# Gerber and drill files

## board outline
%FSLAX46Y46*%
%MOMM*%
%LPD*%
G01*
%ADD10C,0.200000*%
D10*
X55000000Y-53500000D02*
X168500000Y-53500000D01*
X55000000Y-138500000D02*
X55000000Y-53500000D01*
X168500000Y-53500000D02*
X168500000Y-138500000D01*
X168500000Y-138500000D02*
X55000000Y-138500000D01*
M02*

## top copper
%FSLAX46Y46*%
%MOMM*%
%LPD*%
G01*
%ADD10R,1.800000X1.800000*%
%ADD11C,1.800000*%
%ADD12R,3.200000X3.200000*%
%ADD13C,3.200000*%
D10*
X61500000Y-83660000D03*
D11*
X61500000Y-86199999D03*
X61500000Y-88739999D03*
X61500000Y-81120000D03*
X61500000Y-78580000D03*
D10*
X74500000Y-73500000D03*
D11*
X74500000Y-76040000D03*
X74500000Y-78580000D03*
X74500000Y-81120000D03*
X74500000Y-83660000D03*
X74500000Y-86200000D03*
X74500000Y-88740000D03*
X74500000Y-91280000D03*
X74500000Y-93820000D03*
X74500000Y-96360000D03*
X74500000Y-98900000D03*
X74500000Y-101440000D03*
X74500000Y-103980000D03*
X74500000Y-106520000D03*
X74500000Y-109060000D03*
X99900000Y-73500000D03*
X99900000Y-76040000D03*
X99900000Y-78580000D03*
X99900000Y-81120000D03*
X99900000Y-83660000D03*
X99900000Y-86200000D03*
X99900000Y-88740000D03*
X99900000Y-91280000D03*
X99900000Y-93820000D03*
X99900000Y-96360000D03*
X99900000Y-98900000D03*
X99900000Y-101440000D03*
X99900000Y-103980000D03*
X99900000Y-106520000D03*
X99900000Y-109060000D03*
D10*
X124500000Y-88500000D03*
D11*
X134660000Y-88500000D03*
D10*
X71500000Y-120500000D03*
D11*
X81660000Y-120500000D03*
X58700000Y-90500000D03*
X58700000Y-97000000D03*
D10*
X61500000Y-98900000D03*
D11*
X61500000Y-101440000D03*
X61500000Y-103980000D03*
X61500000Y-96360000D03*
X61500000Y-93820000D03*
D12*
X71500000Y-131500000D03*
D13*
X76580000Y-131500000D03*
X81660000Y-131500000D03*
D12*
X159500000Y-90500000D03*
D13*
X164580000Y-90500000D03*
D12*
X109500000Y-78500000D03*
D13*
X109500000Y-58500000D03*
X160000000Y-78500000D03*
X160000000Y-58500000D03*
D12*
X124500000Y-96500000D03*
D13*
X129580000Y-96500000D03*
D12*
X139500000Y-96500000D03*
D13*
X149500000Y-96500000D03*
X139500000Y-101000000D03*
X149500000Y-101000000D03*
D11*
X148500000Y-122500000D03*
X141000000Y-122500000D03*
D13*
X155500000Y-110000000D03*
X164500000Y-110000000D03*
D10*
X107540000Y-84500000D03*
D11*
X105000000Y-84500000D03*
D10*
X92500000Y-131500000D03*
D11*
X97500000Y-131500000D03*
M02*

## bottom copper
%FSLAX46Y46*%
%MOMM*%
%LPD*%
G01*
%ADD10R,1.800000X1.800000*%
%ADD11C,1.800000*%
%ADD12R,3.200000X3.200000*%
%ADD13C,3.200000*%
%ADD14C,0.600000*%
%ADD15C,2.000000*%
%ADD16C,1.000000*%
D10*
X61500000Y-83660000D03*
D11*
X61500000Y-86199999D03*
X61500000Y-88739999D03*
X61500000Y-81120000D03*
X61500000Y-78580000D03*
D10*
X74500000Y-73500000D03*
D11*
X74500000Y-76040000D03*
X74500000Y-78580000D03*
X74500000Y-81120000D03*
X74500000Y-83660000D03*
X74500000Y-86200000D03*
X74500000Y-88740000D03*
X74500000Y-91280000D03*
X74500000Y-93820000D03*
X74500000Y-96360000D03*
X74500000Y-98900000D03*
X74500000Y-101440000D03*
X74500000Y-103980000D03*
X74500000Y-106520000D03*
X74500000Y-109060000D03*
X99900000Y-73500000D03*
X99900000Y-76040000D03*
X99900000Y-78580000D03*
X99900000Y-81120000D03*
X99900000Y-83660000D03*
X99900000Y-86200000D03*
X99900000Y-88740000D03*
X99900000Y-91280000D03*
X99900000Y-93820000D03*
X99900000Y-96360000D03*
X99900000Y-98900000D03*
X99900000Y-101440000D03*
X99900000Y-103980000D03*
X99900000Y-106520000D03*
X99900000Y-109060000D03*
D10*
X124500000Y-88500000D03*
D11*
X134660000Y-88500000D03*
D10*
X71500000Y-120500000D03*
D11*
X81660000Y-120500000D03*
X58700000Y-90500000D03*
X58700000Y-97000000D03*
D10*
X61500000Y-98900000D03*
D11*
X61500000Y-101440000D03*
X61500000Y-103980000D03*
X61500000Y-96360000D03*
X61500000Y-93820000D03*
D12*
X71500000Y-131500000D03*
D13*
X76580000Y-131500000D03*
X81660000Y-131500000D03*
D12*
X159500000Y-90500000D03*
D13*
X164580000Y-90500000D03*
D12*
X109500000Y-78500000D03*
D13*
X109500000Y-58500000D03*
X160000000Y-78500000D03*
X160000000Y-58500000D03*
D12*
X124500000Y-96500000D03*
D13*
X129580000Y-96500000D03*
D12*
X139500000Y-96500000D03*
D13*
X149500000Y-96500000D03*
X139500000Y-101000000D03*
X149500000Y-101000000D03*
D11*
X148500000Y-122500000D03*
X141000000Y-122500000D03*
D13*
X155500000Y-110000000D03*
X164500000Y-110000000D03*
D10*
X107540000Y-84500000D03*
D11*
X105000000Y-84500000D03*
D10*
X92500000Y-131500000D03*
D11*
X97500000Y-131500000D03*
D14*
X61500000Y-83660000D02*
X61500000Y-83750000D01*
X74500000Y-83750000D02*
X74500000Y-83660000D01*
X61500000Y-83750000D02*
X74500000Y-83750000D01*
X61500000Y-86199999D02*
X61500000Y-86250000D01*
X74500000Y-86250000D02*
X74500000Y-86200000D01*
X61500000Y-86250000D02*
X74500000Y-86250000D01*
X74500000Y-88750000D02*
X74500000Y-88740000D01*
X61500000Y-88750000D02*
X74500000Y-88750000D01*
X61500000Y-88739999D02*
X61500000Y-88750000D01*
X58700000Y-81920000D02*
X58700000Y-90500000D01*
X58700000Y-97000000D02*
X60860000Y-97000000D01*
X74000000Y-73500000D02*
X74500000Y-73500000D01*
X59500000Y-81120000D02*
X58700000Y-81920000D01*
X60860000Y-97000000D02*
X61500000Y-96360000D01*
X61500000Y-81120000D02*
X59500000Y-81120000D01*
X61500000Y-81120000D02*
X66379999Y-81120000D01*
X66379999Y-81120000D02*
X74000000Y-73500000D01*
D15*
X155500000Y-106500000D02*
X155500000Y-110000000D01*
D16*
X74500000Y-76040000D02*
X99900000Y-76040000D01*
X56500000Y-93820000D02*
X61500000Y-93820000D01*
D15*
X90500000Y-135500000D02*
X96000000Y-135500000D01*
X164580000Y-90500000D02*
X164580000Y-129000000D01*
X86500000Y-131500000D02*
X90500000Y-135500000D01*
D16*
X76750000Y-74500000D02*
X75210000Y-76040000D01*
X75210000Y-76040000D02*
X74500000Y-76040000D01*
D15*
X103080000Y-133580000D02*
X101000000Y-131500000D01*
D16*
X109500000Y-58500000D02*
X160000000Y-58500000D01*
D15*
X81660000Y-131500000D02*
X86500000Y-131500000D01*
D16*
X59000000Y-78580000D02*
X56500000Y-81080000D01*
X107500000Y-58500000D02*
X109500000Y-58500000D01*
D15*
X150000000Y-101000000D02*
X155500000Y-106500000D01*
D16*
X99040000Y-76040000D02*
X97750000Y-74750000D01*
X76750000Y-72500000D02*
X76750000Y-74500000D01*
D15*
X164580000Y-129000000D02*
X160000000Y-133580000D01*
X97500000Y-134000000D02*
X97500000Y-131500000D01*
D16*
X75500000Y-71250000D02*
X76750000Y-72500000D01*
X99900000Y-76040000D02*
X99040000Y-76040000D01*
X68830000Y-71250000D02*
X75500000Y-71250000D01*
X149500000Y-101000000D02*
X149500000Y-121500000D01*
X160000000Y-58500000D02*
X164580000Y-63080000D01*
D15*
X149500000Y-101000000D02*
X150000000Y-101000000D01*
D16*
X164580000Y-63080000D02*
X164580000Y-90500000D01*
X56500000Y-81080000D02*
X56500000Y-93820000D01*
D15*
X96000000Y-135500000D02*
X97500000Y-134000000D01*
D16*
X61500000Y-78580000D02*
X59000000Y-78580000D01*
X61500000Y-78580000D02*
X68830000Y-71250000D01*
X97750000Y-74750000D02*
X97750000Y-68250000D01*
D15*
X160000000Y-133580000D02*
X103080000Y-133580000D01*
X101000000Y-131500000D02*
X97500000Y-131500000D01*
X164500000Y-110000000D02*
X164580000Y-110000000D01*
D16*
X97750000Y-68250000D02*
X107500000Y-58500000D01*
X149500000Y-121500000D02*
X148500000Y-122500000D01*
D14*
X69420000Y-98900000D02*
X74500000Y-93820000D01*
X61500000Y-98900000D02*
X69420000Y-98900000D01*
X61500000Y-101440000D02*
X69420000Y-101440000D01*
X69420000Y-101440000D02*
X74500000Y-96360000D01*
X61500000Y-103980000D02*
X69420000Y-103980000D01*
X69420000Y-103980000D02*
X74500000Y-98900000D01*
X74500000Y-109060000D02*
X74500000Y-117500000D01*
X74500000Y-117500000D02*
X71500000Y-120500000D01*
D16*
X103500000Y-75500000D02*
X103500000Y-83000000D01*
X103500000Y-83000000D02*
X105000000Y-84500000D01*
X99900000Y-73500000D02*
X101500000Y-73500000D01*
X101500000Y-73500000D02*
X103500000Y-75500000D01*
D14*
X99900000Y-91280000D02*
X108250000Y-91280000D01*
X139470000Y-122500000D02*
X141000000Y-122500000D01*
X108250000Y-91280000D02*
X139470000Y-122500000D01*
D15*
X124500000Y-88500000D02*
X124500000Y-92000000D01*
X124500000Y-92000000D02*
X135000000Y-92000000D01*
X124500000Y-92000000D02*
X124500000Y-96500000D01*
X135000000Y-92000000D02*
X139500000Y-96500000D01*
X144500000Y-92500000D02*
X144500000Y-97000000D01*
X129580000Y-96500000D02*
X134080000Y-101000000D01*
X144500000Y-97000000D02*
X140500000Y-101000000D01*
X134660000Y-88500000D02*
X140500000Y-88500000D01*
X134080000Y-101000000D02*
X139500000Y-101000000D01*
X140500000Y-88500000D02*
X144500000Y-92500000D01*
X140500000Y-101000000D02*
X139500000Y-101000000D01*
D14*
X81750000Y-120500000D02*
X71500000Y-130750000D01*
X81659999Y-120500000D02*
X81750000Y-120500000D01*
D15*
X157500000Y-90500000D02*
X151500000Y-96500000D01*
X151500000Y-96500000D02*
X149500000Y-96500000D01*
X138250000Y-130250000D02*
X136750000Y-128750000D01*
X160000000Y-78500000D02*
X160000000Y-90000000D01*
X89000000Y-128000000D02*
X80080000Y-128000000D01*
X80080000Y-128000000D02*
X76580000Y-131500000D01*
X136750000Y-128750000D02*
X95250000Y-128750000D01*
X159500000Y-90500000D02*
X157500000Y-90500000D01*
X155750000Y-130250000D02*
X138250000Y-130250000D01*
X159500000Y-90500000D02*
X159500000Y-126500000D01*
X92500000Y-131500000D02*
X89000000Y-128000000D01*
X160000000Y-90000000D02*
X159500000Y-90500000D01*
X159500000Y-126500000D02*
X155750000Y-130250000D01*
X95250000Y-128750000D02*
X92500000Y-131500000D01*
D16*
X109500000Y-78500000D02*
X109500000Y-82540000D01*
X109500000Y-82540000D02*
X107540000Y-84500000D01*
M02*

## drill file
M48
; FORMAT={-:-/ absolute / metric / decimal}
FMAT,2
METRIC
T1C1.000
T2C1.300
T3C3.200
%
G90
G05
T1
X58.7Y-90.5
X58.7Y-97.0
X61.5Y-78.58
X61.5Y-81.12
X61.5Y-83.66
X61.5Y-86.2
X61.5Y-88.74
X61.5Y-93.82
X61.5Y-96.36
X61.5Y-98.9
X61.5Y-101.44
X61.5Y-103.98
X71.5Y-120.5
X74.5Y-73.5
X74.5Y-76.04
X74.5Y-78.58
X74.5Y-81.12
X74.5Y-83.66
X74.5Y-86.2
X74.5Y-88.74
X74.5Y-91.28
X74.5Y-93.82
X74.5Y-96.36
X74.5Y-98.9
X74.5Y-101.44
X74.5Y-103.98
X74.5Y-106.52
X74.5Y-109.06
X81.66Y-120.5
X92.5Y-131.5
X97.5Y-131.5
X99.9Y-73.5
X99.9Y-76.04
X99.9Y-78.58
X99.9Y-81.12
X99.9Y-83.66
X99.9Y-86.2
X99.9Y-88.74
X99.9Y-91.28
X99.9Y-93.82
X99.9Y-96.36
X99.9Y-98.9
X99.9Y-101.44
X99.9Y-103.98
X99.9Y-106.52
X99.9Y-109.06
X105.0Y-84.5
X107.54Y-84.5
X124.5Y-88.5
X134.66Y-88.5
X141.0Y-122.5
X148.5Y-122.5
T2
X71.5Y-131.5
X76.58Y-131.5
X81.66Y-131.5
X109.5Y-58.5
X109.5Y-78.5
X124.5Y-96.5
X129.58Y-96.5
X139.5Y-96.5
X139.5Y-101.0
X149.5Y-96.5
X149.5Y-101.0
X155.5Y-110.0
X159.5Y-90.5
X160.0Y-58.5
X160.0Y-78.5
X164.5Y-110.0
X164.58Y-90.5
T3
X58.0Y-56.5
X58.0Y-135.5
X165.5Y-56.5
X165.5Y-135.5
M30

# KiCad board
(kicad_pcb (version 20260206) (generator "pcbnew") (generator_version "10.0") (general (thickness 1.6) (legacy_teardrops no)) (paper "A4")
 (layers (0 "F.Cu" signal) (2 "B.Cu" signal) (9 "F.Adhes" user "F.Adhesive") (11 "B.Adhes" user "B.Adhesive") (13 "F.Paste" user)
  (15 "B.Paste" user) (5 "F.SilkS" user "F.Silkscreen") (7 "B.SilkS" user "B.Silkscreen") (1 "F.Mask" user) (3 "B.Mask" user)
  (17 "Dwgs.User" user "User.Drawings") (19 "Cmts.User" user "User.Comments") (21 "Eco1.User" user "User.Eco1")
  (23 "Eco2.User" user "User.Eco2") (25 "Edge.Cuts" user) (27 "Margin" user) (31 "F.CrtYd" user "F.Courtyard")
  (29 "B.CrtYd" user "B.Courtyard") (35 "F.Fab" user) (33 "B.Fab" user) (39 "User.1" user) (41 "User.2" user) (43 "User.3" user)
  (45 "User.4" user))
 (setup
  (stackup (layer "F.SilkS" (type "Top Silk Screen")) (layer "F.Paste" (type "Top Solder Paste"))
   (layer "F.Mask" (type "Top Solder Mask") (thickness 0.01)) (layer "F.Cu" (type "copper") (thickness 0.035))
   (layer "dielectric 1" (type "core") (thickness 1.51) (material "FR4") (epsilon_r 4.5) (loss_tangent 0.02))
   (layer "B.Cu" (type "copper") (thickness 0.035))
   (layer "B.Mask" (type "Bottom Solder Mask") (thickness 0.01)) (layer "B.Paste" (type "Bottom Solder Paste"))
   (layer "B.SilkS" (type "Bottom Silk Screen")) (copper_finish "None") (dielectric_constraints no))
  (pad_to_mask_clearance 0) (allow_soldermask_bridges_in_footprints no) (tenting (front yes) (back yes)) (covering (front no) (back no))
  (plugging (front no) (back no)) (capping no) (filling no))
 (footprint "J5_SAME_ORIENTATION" (layer "F.Cu") (at 61.5 83.5 -90)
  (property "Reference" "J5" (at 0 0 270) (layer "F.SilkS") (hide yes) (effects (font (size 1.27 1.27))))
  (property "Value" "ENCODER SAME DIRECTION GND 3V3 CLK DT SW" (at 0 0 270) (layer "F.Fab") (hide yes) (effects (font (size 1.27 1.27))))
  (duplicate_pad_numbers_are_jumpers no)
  (pad "1" thru_hole rect (at 0.16 0 270) (size 1.8 1.8) (drill 1) (layers "*.Cu") (remove_unused_layers no) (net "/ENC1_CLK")
   (clearance 0.5) (thermal_bridge_angle 45))
  (pad "2" thru_hole circle (at 2.699999 0 270) (size 1.8 1.8) (drill 1) (layers "*.Cu") (remove_unused_layers no) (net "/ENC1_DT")
   (clearance 0.5))
  (pad "3" thru_hole circle (at 5.239999 0 270) (size 1.8 1.8) (drill 1) (layers "*.Cu") (remove_unused_layers no) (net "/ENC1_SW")
   (clearance 0.5))
  (pad "4" thru_hole circle (at -2.38 0 270) (size 1.8 1.8) (drill 1) (layers "*.Cu") (remove_unused_layers no) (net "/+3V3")
   (clearance 0.5))
  (pad "5" thru_hole circle (at -4.92 0 270) (size 1.8 1.8) (drill 1) (layers "*.Cu") (remove_unused_layers no) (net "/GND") (clearance 0.5)))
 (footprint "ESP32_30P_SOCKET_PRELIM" (layer "F.Cu") (at 74.5 73.5)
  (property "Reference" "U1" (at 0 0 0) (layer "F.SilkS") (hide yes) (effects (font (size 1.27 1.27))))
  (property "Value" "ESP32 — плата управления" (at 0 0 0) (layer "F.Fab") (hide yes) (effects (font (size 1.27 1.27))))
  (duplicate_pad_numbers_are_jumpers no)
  (pad "1" thru_hole rect (at 0 0) (size 1.8 1.8) (drill 1) (layers "*.Cu") (remove_unused_layers no) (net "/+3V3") (clearance 0.5)
   (thermal_bridge_angle 45))
  (pad "2" thru_hole circle (at 0 2.54) (size 1.8 1.8) (drill 1) (layers "*.Cu") (remove_unused_layers no) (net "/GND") (clearance 0.5))
  (pad "3" thru_hole circle (at 0 5.08) (size 1.8 1.8) (drill 1) (layers "*.Cu") (remove_unused_layers no) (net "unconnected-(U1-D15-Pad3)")
   (clearance 0.5))
  (pad "4" thru_hole circle (at 0 7.62) (size 1.8 1.8) (drill 1) (layers "*.Cu") (remove_unused_layers no) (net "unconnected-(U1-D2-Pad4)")
   (clearance 0.5))
  (pad "5" thru_hole circle (at 0 10.16) (size 1.8 1.8) (drill 1) (layers "*.Cu") (remove_unused_layers no) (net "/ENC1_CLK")
   (clearance 0.5))
  (pad "6" thru_hole circle (at 0 12.7) (size 1.8 1.8) (drill 1) (layers "*.Cu") (remove_unused_layers no) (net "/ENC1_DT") (clearance 0.5))
  (pad "7" thru_hole circle (at 0 15.24) (size 1.8 1.8) (drill 1) (layers "*.Cu") (remove_unused_layers no) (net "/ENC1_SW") (clearance 0.5))
  (pad "8" thru_hole circle (at 0 17.78) (size 1.8 1.8) (drill 1) (layers "*.Cu") (remove_unused_layers no) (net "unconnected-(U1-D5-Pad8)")
   (clearance 0.5))
  (pad "9" thru_hole circle (at 0 20.32) (size 1.8 1.8) (drill 1) (layers "*.Cu") (remove_unused_layers no) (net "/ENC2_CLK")
   (clearance 0.5))
  (pad "10" thru_hole circle (at 0 22.86) (size 1.8 1.8) (drill 1) (layers "*.Cu") (remove_unused_layers no) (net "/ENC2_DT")
   (clearance 0.5))
  (pad "11" thru_hole circle (at 0 25.4) (size 1.8 1.8) (drill 1) (layers "*.Cu") (remove_unused_layers no) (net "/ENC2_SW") (clearance 0.5))
  (pad "12" thru_hole circle (at 0 27.94) (size 1.8 1.8) (drill 1) (layers "*.Cu") (remove_unused_layers no)
   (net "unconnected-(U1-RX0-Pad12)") (clearance 0.5))
  (pad "13" thru_hole circle (at 0 30.48) (size 1.8 1.8) (drill 1) (layers "*.Cu") (remove_unused_layers no)
   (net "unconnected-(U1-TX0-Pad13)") (clearance 0.5))
  (pad "14" thru_hole circle (at 0 33.02) (size 1.8 1.8) (drill 1) (layers "*.Cu") (remove_unused_layers no)
   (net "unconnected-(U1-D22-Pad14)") (clearance 0.5))
  (pad "15" thru_hole circle (at 0 35.56) (size 1.8 1.8) (drill 1) (layers "*.Cu") (remove_unused_layers no) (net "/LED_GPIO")
   (clearance 0.5))
  (pad "16" thru_hole circle (at 25.4 0) (size 1.8 1.8) (drill 1) (layers "*.Cu") (remove_unused_layers no) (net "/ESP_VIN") (clearance 0.5))
  (pad "17" thru_hole circle (at 25.4 2.54) (size 1.8 1.8) (drill 1) (layers "*.Cu") (remove_unused_layers no) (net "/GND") (clearance 0.5))
  (pad "18" thru_hole circle (at 25.4 5.08) (size 1.8 1.8) (drill 1) (layers "*.Cu") (remove_unused_layers no)
   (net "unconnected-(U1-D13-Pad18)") (clearance 0.5))
  (pad "19" thru_hole circle (at 25.4 7.62) (size 1.8 1.8) (drill 1) (layers "*.Cu") (remove_unused_layers no)
   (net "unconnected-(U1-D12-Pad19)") (clearance 0.5))
  (pad "20" thru_hole circle (at 25.4 10.16) (size 1.8 1.8) (drill 1) (layers "*.Cu") (remove_unused_layers no)
   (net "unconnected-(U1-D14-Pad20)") (clearance 0.5))
  (pad "21" thru_hole circle (at 25.4 12.7) (size 1.8 1.8) (drill 1) (layers "*.Cu") (remove_unused_layers no)
   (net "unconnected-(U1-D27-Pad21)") (clearance 0.5))
  (pad "22" thru_hole circle (at 25.4 15.24) (size 1.8 1.8) (drill 1) (layers "*.Cu") (remove_unused_layers no)
   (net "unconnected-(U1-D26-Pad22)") (clearance 0.5))
  (pad "23" thru_hole circle (at 25.4 17.78) (size 1.8 1.8) (drill 1) (layers "*.Cu") (remove_unused_layers no) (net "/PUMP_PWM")
   (clearance 0.5))
  (pad "24" thru_hole circle (at 25.4 20.32) (size 1.8 1.8) (drill 1) (layers "*.Cu") (remove_unused_layers no)
   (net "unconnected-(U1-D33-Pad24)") (clearance 0.5))
  (pad "25" thru_hole circle (at 25.4 22.86) (size 1.8 1.8) (drill 1) (layers "*.Cu") (remove_unused_layers no)
   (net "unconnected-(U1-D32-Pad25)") (clearance 0.5))
  (pad "26" thru_hole circle (at 25.4 25.4) (size 1.8 1.8) (drill 1) (layers "*.Cu") (remove_unused_layers no)
   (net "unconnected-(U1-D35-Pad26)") (clearance 0.5))
  (pad "27" thru_hole circle (at 25.4 27.94) (size 1.8 1.8) (drill 1) (layers "*.Cu") (remove_unused_layers no)
   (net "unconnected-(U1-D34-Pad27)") (clearance 0.5))
  (pad "28" thru_hole circle (at 25.4 30.48) (size 1.8 1.8) (drill 1) (layers "*.Cu") (remove_unused_layers no)
   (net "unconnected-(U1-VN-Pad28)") (clearance 0.5))
  (pad "29" thru_hole circle (at 25.4 33.02) (size 1.8 1.8) (drill 1) (layers "*.Cu") (remove_unused_layers no)
   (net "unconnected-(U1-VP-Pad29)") (clearance 0.5))
  (pad "30" thru_hole circle (at 25.4 35.56) (size 1.8 1.8) (drill 1) (layers "*.Cu") (remove_unused_layers no)
   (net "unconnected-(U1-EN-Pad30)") (clearance 0.5)))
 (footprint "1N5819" (layer "F.Cu") (at 124.5 88.5)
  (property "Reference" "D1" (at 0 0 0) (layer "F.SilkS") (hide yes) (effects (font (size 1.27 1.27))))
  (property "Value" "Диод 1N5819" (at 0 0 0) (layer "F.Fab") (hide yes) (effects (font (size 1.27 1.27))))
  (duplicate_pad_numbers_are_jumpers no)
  (pad "1" thru_hole rect (at 0 0) (size 1.8 1.8) (drill 1) (layers "*.Cu") (remove_unused_layers no) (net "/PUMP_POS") (clearance 0.5)
   (thermal_bridge_angle 45))
  (pad "2" thru_hole circle (at 10.16 0) (size 1.8 1.8) (drill 1) (layers "*.Cu") (remove_unused_layers no) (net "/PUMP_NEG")
   (clearance 0.5)))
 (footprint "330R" (layer "F.Cu") (at 71.5 120.5)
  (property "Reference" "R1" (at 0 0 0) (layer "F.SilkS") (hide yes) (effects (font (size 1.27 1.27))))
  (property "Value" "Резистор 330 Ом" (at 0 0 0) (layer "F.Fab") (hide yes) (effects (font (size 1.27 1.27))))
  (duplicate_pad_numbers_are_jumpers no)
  (pad "1" thru_hole rect (at 0 0) (size 1.8 1.8) (drill 1) (layers "*.Cu") (remove_unused_layers no) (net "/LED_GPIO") (clearance 0.5)
   (thermal_bridge_angle 45))
  (pad "2" thru_hole circle (at 10.16 0) (size 1.8 1.8) (drill 1) (layers "*.Cu") (remove_unused_layers no) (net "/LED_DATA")
   (clearance 0.5)))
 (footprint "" (layer "F.Cu") (at 58 135.5)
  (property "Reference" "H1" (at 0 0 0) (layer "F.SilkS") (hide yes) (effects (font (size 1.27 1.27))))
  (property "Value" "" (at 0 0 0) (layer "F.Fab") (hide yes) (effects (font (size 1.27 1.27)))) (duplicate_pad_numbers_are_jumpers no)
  (pad "" np_thru_hole circle (at 0 0) (size 3.2 3.2) (drill 3.2) (layers "*.Cu") (clearance 0.5)))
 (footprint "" (layer "F.Cu") (at 58.7 90.5)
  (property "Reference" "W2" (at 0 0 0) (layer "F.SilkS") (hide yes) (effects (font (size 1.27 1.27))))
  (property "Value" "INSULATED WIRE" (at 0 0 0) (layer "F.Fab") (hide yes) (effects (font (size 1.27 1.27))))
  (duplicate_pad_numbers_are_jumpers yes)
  (pad "1" thru_hole circle (at 0 0) (size 1.8 1.8) (drill 1) (layers "*.Cu") (remove_unused_layers no) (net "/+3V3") (clearance 0.5))
  (pad "1" thru_hole circle (at 0 6.5) (size 1.8 1.8) (drill 1) (layers "*.Cu") (remove_unused_layers no) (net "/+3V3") (clearance 0.5)))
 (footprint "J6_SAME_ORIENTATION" (layer "F.Cu") (at 61.5 96.5 -90)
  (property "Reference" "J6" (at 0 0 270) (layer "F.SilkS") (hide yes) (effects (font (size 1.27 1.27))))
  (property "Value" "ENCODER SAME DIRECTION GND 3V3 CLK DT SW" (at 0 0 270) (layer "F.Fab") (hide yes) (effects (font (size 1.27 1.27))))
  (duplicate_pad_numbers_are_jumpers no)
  (pad "1" thru_hole rect (at 2.4 0 270) (size 1.8 1.8) (drill 1) (layers "*.Cu") (remove_unused_layers no) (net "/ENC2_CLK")
   (clearance 0.5) (thermal_bridge_angle 45))
  (pad "2" thru_hole circle (at 4.94 0 270) (size 1.8 1.8) (drill 1) (layers "*.Cu") (remove_unused_layers no) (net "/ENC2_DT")
   (clearance 0.5))
  (pad "3" thru_hole circle (at 7.48 0 270) (size 1.8 1.8) (drill 1) (layers "*.Cu") (remove_unused_layers no) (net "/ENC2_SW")
   (clearance 0.5))
  (pad "4" thru_hole circle (at -0.14 0 270) (size 1.8 1.8) (drill 1) (layers "*.Cu") (remove_unused_layers no) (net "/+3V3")
   (clearance 0.5))
  (pad "5" thru_hole circle (at -2.68 0 270) (size 1.8 1.8) (drill 1) (layers "*.Cu") (remove_unused_layers no) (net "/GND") (clearance 0.5)))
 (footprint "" (layer "F.Cu") (at 58 56.5)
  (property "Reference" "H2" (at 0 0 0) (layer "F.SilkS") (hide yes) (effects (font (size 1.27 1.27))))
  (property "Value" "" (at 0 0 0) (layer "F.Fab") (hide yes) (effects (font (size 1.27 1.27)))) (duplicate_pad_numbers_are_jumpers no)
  (pad "" np_thru_hole circle (at 0 0) (size 3.2 3.2) (drill 3.2) (layers "*.Cu") (clearance 0.5)))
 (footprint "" (layer "F.Cu") (at 165.5 135.5)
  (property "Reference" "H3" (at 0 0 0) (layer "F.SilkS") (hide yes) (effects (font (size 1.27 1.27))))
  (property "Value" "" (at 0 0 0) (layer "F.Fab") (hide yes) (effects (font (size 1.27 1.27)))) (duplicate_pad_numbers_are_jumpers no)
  (pad "" np_thru_hole circle (at 0 0) (size 3.2 3.2) (drill 3.2) (layers "*.Cu") (clearance 0.5)))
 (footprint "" (layer "F.Cu") (at 165.5 56.5)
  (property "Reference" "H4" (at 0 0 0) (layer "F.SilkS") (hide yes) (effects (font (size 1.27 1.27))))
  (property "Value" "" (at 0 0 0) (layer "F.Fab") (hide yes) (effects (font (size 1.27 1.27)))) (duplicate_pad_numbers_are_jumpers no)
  (pad "" np_thru_hole circle (at 0 0) (size 3.2 3.2) (drill 3.2) (layers "*.Cu") (clearance 0.5)))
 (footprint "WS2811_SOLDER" (layer "F.Cu") (at 71.5 131.5)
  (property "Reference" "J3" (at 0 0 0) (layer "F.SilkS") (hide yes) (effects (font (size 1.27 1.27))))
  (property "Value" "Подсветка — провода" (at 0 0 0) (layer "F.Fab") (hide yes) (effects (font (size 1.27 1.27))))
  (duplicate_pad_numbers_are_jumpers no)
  (pad "1" thru_hole rect (at 0 0) (size 3.2 3.2) (drill 1.3) (layers "*.Cu") (remove_unused_layers no) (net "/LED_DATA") (clearance 0.5)
   (thermal_bridge_angle 45))
  (pad "2" thru_hole circle (at 5.08 0) (size 3.2 3.2) (drill 1.3) (layers "*.Cu") (remove_unused_layers no) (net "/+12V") (clearance 0.5))
  (pad "3" thru_hole circle (at 10.16 0) (size 3.2 3.2) (drill 1.3) (layers "*.Cu") (remove_unused_layers no) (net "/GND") (clearance 0.5)))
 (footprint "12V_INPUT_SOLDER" (layer "F.Cu") (at 159.5 90.5)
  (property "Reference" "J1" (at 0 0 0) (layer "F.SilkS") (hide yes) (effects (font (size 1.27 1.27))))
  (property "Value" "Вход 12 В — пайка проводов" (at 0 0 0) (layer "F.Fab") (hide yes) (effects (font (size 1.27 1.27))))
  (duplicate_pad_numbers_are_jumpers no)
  (pad "1" thru_hole rect (at 0 0) (size 3.2 3.2) (drill 1.3) (layers "*.Cu") (remove_unused_layers no) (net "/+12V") (clearance 0.5)
   (thermal_bridge_angle 45))
  (pad "2" thru_hole circle (at 5.08 0) (size 3.2 3.2) (drill 1.3) (layers "*.Cu") (remove_unused_layers no) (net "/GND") (clearance 0.5)))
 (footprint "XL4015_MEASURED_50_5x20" (layer "F.Cu") (at 109.5 78.5 90)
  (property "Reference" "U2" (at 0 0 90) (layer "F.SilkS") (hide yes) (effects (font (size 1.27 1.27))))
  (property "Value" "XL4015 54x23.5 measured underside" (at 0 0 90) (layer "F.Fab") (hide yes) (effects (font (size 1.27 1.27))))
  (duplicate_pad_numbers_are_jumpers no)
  (pad "1" thru_hole rect (at 0 0 90) (size 3.2 3.2) (drill 1.3) (layers "*.Cu") (remove_unused_layers no) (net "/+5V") (clearance 0.5)
   (thermal_bridge_angle 45))
  (pad "2" thru_hole circle (at 20 0 90) (size 3.2 3.2) (drill 1.3) (layers "*.Cu") (remove_unused_layers no) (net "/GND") (clearance 0.5))
  (pad "3" thru_hole circle (at 0 50.5 90) (size 3.2 3.2) (drill 1.3) (layers "*.Cu") (remove_unused_layers no) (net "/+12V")
   (clearance 0.5))
  (pad "4" thru_hole circle (at 20 50.5 90) (size 3.2 3.2) (drill 1.3) (layers "*.Cu") (remove_unused_layers no) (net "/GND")
   (clearance 0.5)))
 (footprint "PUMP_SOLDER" (layer "F.Cu") (at 124.5 96.5)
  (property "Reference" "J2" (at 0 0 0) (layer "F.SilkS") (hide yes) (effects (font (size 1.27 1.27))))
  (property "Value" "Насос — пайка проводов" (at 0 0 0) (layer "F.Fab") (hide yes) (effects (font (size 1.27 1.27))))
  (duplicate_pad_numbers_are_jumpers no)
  (pad "1" thru_hole rect (at 0 0) (size 3.2 3.2) (drill 1.3) (layers "*.Cu") (remove_unused_layers no) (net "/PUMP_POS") (clearance 0.5)
   (thermal_bridge_angle 45))
  (pad "2" thru_hole circle (at 5.08 0) (size 3.2 3.2) (drill 1.3) (layers "*.Cu") (remove_unused_layers no) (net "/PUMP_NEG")
   (clearance 0.5)))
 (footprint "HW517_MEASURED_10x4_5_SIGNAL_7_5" (layer "F.Cu") (at 139.5 96.5)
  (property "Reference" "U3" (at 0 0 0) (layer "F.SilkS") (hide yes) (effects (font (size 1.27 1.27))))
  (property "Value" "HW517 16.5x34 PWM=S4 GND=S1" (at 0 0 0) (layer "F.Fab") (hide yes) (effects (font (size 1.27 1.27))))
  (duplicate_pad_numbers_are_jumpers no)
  (pad "1" thru_hole rect (at 0 0) (size 3.2 3.2) (drill 1.3) (layers "*.Cu") (remove_unused_layers no) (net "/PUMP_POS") (clearance 0.5)
   (thermal_bridge_angle 45))
  (pad "2" thru_hole circle (at 10 0) (size 3.2 3.2) (drill 1.3) (layers "*.Cu") (remove_unused_layers no) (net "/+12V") (clearance 0.5))
  (pad "3" thru_hole circle (at 0 4.5) (size 3.2 3.2) (drill 1.3) (layers "*.Cu") (remove_unused_layers no) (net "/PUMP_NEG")
   (clearance 0.5))
  (pad "4" thru_hole circle (at 10 4.5) (size 3.2 3.2) (drill 1.3) (layers "*.Cu") (remove_unused_layers no) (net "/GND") (clearance 0.5))
  (pad "5" thru_hole circle (at 9 26) (size 1.8 1.8) (drill 1) (layers "*.Cu") (remove_unused_layers no) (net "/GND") (clearance 0.5))
  (pad "6" thru_hole circle (at 1.5 26) (size 1.8 1.8) (drill 1) (layers "*.Cu") (remove_unused_layers no) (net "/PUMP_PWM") (clearance 0.5)))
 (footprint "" (layer "F.Cu") (at 155.5 110)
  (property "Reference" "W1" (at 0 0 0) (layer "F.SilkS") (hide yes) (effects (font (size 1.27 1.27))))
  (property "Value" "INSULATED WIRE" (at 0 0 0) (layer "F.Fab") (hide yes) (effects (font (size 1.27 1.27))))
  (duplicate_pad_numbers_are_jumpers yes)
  (pad "1" thru_hole circle (at 0 0) (size 3.2 3.2) (drill 1.3) (layers "*.Cu") (remove_unused_layers no) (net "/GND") (clearance 0.5))
  (pad "1" thru_hole circle (at 9 0) (size 3.2 3.2) (drill 1.3) (layers "*.Cu") (remove_unused_layers no) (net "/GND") (clearance 0.5)))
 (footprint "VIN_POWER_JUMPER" (layer "F.Cu") (at 107.54 84.5)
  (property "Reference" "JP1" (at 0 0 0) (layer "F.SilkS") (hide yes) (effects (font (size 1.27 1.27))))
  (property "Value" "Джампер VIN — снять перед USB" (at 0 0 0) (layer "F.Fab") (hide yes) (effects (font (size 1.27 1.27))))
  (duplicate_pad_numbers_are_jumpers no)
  (pad "1" thru_hole rect (at 0 0) (size 1.8 1.8) (drill 1) (layers "*.Cu") (remove_unused_layers no) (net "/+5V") (clearance 0.5)
   (thermal_bridge_angle 45))
  (pad "2" thru_hole circle (at -2.54 0) (size 1.8 1.8) (drill 1) (layers "*.Cu") (remove_unused_layers no) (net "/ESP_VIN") (clearance 0.5)))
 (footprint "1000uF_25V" (layer "F.Cu") (at 92.5 131.5)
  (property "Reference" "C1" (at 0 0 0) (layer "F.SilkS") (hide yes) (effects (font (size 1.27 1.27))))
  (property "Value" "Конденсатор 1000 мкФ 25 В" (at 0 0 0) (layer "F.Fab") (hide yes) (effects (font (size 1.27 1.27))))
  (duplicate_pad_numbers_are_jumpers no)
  (pad "1" thru_hole rect (at 0 0) (size 1.8 1.8) (drill 1) (layers "*.Cu") (remove_unused_layers no) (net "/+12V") (clearance 0.5)
   (thermal_bridge_angle 45))
  (pad "2" thru_hole circle (at 5 0) (size 1.8 1.8) (drill 1) (layers "*.Cu") (remove_unused_layers no) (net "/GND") (clearance 0.5)))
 (gr_line (start 55 53.5) (end 168.5 53.5) (stroke (width 0.2) (type default)) (layer "Edge.Cuts"))
 (gr_line (start 55 138.5) (end 55 53.5) (stroke (width 0.2) (type default)) (layer "Edge.Cuts"))
 (gr_line (start 168.5 53.5) (end 168.5 138.5) (stroke (width 0.2) (type default)) (layer "Edge.Cuts"))
 (gr_line (start 168.5 138.5) (end 55 138.5) (stroke (width 0.2) (type default)) (layer "Edge.Cuts"))
 (segment (start 61.5 83.66) (end 61.5 83.75) (width 0.6) (layer "B.Cu") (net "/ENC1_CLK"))
 (segment (start 74.5 83.75) (end 74.5 83.66) (width 0.6) (layer "B.Cu") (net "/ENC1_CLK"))
 (segment (start 61.5 83.75) (end 74.5 83.75) (width 0.6) (layer "B.Cu") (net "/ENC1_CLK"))
 (segment (start 61.5 86.199999) (end 61.5 86.25) (width 0.6) (layer "B.Cu") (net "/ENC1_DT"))
 (segment (start 74.5 86.25) (end 74.5 86.2) (width 0.6) (layer "B.Cu") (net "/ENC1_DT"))
 (segment (start 61.5 86.25) (end 74.5 86.25) (width 0.6) (layer "B.Cu") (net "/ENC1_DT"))
 (segment (start 74.5 88.75) (end 74.5 88.74) (width 0.6) (layer "B.Cu") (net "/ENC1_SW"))
 (segment (start 61.5 88.75) (end 74.5 88.75) (width 0.6) (layer "B.Cu") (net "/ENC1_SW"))
 (segment (start 61.5 88.739999) (end 61.5 88.75) (width 0.6) (layer "B.Cu") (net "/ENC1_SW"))
 (segment (start 58.7 81.92) (end 58.7 90.5) (width 0.6) (layer "B.Cu") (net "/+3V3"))
 (segment (start 58.7 97) (end 60.86 97) (width 0.6) (layer "B.Cu") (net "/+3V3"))
 (segment (start 74 73.5) (end 74.5 73.5) (width 0.6) (layer "B.Cu") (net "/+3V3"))
 (segment (start 59.5 81.12) (end 58.7 81.92) (width 0.6) (layer "B.Cu") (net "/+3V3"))
 (segment (start 60.86 97) (end 61.5 96.36) (width 0.6) (layer "B.Cu") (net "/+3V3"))
 (segment (start 61.5 81.12) (end 59.5 81.12) (width 0.6) (layer "B.Cu") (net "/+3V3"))
 (segment (start 61.5 81.12) (end 66.379999 81.12) (width 0.6) (layer "B.Cu") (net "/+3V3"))
 (segment (start 66.379999 81.12) (end 74 73.5) (width 0.6) (layer "B.Cu") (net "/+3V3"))
 (segment (start 155.5 106.5) (end 155.5 110) (width 2) (layer "B.Cu") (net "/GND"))
 (segment (start 74.5 76.04) (end 99.9 76.04) (width 1) (layer "B.Cu") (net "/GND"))
 (segment (start 56.5 93.82) (end 61.5 93.82) (width 1) (layer "B.Cu") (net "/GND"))
 (segment (start 90.5 135.5) (end 96 135.5) (width 2) (layer "B.Cu") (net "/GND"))
 (segment (start 164.58 90.5) (end 164.58 129) (width 2) (layer "B.Cu") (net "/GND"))
 (segment (start 86.5 131.5) (end 90.5 135.5) (width 2) (layer "B.Cu") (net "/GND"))
 (segment (start 76.75 74.5) (end 75.21 76.04) (width 1) (layer "B.Cu") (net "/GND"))
 (segment (start 75.21 76.04) (end 74.5 76.04) (width 1) (layer "B.Cu") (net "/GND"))
 (segment (start 103.08 133.58) (end 101 131.5) (width 2) (layer "B.Cu") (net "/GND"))
 (segment (start 109.5 58.5) (end 160 58.5) (width 1) (layer "B.Cu") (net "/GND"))
 (segment (start 81.66 131.5) (end 86.5 131.5) (width 2) (layer "B.Cu") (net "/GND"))
 (segment (start 59 78.58) (end 56.5 81.08) (width 1) (layer "B.Cu") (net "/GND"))
 (segment (start 107.5 58.5) (end 109.5 58.5) (width 1) (layer "B.Cu") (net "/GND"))
 (segment (start 150 101) (end 155.5 106.5) (width 2) (layer "B.Cu") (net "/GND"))
 (segment (start 99.04 76.04) (end 97.75 74.75) (width 1) (layer "B.Cu") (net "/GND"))
 (segment (start 76.75 72.5) (end 76.75 74.5) (width 1) (layer "B.Cu") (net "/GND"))
 (segment (start 164.58 129) (end 160 133.58) (width 2) (layer "B.Cu") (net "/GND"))
 (segment (start 97.5 134) (end 97.5 131.5) (width 2) (layer "B.Cu") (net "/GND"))
 (segment (start 75.5 71.25) (end 76.75 72.5) (width 1) (layer "B.Cu") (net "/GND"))
 (segment (start 99.9 76.04) (end 99.04 76.04) (width 1) (layer "B.Cu") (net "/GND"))
 (segment (start 68.83 71.25) (end 75.5 71.25) (width 1) (layer "B.Cu") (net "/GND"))
 (segment (start 149.5 101) (end 149.5 121.5) (width 1) (layer "B.Cu") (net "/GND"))
 (segment (start 160 58.5) (end 164.58 63.08) (width 1) (layer "B.Cu") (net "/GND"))
 (segment (start 149.5 101) (end 150 101) (width 2) (layer "B.Cu") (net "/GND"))
 (segment (start 164.58 63.08) (end 164.58 90.5) (width 1) (layer "B.Cu") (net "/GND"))
 (segment (start 56.5 81.08) (end 56.5 93.82) (width 1) (layer "B.Cu") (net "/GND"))
 (segment (start 96 135.5) (end 97.5 134) (width 2) (layer "B.Cu") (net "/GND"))
 (segment (start 61.5 78.58) (end 59 78.58) (width 1) (layer "B.Cu") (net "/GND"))
 (segment (start 61.5 78.58) (end 68.83 71.25) (width 1) (layer "B.Cu") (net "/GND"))
 (segment (start 97.75 74.75) (end 97.75 68.25) (width 1) (layer "B.Cu") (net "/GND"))
 (segment (start 160 133.58) (end 103.08 133.58) (width 2) (layer "B.Cu") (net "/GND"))
 (segment (start 101 131.5) (end 97.5 131.5) (width 2) (layer "B.Cu") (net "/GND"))
 (segment (start 164.5 110) (end 164.58 110) (width 2) (layer "B.Cu") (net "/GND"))
 (segment (start 97.75 68.25) (end 107.5 58.5) (width 1) (layer "B.Cu") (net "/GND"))
 (segment (start 149.5 121.5) (end 148.5 122.5) (width 1) (layer "B.Cu") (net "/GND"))
 (segment (start 69.42 98.9) (end 74.5 93.82) (width 0.6) (layer "B.Cu") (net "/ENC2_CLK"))
 (segment (start 61.5 98.9) (end 69.42 98.9) (width 0.6) (layer "B.Cu") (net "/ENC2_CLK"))
 (segment (start 61.5 101.44) (end 69.42 101.44) (width 0.6) (layer "B.Cu") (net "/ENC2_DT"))
 (segment (start 69.42 101.44) (end 74.5 96.36) (width 0.6) (layer "B.Cu") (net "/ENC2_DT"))
 (segment (start 61.5 103.98) (end 69.42 103.98) (width 0.6) (layer "B.Cu") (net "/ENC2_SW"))
 (segment (start 69.42 103.98) (end 74.5 98.9) (width 0.6) (layer "B.Cu") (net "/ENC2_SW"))
 (segment (start 74.5 109.06) (end 74.5 117.5) (width 0.6) (layer "B.Cu") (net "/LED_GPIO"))
 (segment (start 74.5 117.5) (end 71.5 120.5) (width 0.6) (layer "B.Cu") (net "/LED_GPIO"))
 (segment (start 103.5 75.5) (end 103.5 83) (width 1) (layer "B.Cu") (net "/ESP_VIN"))
 (segment (start 103.5 83) (end 105 84.5) (width 1) (layer "B.Cu") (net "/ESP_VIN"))
 (segment (start 99.9 73.5) (end 101.5 73.5) (width 1) (layer "B.Cu") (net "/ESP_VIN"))
 (segment (start 101.5 73.5) (end 103.5 75.5) (width 1) (layer "B.Cu") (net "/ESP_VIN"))
 (segment (start 99.9 91.28) (end 108.25 91.28) (width 0.6) (layer "B.Cu") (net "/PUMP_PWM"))
 (segment (start 139.47 122.5) (end 141 122.5) (width 0.6) (layer "B.Cu") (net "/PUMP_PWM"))
 (segment (start 108.25 91.28) (end 139.47 122.5) (width 0.6) (layer "B.Cu") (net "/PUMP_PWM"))
 (segment (start 124.5 88.5) (end 124.5 92) (width 2) (layer "B.Cu") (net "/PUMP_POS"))
 (segment (start 124.5 92) (end 135 92) (width 2) (layer "B.Cu") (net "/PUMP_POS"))
 (segment (start 124.5 92) (end 124.5 96.5) (width 2) (layer "B.Cu") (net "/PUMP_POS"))
 (segment (start 135 92) (end 139.5 96.5) (width 2) (layer "B.Cu") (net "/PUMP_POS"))
 (segment (start 144.5 92.5) (end 144.5 97) (width 2) (layer "B.Cu") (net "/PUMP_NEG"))
 (segment (start 129.58 96.5) (end 134.08 101) (width 2) (layer "B.Cu") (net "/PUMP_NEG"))
 (segment (start 144.5 97) (end 140.5 101) (width 2) (layer "B.Cu") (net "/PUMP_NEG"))
 (segment (start 134.66 88.5) (end 140.5 88.5) (width 2) (layer "B.Cu") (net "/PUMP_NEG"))
 (segment (start 134.08 101) (end 139.5 101) (width 2) (layer "B.Cu") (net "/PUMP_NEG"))
 (segment (start 140.5 88.5) (end 144.5 92.5) (width 2) (layer "B.Cu") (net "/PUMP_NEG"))
 (segment (start 140.5 101) (end 139.5 101) (width 2) (layer "B.Cu") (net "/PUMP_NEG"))
 (segment (start 81.75 120.5) (end 71.5 130.75) (width 0.6) (layer "B.Cu") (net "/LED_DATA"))
 (segment (start 81.659999 120.5) (end 81.75 120.5) (width 0.6) (layer "B.Cu") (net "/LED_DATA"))
 (segment (start 157.5 90.5) (end 151.5 96.5) (width 2) (layer "B.Cu") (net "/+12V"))
 (segment (start 151.5 96.5) (end 149.5 96.5) (width 2) (layer "B.Cu") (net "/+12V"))
 (segment (start 138.25 130.25) (end 136.75 128.75) (width 2) (layer "B.Cu") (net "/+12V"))
 (segment (start 160 78.5) (end 160 90) (width 2) (layer "B.Cu") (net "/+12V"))
 (segment (start 89 128) (end 80.08 128) (width 2) (layer "B.Cu") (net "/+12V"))
 (segment (start 80.08 128) (end 76.58 131.5) (width 2) (layer "B.Cu") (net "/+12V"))
 (segment (start 136.75 128.75) (end 95.25 128.75) (width 2) (layer "B.Cu") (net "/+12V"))
 (segment (start 159.5 90.5) (end 157.5 90.5) (width 2) (layer "B.Cu") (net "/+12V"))
 (segment (start 155.75 130.25) (end 138.25 130.25) (width 2) (layer "B.Cu") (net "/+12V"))
 (segment (start 159.5 90.5) (end 159.5 126.5) (width 2) (layer "B.Cu") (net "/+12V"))
 (segment (start 92.5 131.5) (end 89 128) (width 2) (layer "B.Cu") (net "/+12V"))
 (segment (start 160 90) (end 159.5 90.5) (width 2) (layer "B.Cu") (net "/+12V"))
 (segment (start 159.5 126.5) (end 155.75 130.25) (width 2) (layer "B.Cu") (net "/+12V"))
 (segment (start 95.25 128.75) (end 92.5 131.5) (width 2) (layer "B.Cu") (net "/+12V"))
 (segment (start 109.5 78.5) (end 109.5 82.54) (width 1) (layer "B.Cu") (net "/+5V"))
 (segment (start 109.5 82.54) (end 107.54 84.5) (width 1) (layer "B.Cu") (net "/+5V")))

